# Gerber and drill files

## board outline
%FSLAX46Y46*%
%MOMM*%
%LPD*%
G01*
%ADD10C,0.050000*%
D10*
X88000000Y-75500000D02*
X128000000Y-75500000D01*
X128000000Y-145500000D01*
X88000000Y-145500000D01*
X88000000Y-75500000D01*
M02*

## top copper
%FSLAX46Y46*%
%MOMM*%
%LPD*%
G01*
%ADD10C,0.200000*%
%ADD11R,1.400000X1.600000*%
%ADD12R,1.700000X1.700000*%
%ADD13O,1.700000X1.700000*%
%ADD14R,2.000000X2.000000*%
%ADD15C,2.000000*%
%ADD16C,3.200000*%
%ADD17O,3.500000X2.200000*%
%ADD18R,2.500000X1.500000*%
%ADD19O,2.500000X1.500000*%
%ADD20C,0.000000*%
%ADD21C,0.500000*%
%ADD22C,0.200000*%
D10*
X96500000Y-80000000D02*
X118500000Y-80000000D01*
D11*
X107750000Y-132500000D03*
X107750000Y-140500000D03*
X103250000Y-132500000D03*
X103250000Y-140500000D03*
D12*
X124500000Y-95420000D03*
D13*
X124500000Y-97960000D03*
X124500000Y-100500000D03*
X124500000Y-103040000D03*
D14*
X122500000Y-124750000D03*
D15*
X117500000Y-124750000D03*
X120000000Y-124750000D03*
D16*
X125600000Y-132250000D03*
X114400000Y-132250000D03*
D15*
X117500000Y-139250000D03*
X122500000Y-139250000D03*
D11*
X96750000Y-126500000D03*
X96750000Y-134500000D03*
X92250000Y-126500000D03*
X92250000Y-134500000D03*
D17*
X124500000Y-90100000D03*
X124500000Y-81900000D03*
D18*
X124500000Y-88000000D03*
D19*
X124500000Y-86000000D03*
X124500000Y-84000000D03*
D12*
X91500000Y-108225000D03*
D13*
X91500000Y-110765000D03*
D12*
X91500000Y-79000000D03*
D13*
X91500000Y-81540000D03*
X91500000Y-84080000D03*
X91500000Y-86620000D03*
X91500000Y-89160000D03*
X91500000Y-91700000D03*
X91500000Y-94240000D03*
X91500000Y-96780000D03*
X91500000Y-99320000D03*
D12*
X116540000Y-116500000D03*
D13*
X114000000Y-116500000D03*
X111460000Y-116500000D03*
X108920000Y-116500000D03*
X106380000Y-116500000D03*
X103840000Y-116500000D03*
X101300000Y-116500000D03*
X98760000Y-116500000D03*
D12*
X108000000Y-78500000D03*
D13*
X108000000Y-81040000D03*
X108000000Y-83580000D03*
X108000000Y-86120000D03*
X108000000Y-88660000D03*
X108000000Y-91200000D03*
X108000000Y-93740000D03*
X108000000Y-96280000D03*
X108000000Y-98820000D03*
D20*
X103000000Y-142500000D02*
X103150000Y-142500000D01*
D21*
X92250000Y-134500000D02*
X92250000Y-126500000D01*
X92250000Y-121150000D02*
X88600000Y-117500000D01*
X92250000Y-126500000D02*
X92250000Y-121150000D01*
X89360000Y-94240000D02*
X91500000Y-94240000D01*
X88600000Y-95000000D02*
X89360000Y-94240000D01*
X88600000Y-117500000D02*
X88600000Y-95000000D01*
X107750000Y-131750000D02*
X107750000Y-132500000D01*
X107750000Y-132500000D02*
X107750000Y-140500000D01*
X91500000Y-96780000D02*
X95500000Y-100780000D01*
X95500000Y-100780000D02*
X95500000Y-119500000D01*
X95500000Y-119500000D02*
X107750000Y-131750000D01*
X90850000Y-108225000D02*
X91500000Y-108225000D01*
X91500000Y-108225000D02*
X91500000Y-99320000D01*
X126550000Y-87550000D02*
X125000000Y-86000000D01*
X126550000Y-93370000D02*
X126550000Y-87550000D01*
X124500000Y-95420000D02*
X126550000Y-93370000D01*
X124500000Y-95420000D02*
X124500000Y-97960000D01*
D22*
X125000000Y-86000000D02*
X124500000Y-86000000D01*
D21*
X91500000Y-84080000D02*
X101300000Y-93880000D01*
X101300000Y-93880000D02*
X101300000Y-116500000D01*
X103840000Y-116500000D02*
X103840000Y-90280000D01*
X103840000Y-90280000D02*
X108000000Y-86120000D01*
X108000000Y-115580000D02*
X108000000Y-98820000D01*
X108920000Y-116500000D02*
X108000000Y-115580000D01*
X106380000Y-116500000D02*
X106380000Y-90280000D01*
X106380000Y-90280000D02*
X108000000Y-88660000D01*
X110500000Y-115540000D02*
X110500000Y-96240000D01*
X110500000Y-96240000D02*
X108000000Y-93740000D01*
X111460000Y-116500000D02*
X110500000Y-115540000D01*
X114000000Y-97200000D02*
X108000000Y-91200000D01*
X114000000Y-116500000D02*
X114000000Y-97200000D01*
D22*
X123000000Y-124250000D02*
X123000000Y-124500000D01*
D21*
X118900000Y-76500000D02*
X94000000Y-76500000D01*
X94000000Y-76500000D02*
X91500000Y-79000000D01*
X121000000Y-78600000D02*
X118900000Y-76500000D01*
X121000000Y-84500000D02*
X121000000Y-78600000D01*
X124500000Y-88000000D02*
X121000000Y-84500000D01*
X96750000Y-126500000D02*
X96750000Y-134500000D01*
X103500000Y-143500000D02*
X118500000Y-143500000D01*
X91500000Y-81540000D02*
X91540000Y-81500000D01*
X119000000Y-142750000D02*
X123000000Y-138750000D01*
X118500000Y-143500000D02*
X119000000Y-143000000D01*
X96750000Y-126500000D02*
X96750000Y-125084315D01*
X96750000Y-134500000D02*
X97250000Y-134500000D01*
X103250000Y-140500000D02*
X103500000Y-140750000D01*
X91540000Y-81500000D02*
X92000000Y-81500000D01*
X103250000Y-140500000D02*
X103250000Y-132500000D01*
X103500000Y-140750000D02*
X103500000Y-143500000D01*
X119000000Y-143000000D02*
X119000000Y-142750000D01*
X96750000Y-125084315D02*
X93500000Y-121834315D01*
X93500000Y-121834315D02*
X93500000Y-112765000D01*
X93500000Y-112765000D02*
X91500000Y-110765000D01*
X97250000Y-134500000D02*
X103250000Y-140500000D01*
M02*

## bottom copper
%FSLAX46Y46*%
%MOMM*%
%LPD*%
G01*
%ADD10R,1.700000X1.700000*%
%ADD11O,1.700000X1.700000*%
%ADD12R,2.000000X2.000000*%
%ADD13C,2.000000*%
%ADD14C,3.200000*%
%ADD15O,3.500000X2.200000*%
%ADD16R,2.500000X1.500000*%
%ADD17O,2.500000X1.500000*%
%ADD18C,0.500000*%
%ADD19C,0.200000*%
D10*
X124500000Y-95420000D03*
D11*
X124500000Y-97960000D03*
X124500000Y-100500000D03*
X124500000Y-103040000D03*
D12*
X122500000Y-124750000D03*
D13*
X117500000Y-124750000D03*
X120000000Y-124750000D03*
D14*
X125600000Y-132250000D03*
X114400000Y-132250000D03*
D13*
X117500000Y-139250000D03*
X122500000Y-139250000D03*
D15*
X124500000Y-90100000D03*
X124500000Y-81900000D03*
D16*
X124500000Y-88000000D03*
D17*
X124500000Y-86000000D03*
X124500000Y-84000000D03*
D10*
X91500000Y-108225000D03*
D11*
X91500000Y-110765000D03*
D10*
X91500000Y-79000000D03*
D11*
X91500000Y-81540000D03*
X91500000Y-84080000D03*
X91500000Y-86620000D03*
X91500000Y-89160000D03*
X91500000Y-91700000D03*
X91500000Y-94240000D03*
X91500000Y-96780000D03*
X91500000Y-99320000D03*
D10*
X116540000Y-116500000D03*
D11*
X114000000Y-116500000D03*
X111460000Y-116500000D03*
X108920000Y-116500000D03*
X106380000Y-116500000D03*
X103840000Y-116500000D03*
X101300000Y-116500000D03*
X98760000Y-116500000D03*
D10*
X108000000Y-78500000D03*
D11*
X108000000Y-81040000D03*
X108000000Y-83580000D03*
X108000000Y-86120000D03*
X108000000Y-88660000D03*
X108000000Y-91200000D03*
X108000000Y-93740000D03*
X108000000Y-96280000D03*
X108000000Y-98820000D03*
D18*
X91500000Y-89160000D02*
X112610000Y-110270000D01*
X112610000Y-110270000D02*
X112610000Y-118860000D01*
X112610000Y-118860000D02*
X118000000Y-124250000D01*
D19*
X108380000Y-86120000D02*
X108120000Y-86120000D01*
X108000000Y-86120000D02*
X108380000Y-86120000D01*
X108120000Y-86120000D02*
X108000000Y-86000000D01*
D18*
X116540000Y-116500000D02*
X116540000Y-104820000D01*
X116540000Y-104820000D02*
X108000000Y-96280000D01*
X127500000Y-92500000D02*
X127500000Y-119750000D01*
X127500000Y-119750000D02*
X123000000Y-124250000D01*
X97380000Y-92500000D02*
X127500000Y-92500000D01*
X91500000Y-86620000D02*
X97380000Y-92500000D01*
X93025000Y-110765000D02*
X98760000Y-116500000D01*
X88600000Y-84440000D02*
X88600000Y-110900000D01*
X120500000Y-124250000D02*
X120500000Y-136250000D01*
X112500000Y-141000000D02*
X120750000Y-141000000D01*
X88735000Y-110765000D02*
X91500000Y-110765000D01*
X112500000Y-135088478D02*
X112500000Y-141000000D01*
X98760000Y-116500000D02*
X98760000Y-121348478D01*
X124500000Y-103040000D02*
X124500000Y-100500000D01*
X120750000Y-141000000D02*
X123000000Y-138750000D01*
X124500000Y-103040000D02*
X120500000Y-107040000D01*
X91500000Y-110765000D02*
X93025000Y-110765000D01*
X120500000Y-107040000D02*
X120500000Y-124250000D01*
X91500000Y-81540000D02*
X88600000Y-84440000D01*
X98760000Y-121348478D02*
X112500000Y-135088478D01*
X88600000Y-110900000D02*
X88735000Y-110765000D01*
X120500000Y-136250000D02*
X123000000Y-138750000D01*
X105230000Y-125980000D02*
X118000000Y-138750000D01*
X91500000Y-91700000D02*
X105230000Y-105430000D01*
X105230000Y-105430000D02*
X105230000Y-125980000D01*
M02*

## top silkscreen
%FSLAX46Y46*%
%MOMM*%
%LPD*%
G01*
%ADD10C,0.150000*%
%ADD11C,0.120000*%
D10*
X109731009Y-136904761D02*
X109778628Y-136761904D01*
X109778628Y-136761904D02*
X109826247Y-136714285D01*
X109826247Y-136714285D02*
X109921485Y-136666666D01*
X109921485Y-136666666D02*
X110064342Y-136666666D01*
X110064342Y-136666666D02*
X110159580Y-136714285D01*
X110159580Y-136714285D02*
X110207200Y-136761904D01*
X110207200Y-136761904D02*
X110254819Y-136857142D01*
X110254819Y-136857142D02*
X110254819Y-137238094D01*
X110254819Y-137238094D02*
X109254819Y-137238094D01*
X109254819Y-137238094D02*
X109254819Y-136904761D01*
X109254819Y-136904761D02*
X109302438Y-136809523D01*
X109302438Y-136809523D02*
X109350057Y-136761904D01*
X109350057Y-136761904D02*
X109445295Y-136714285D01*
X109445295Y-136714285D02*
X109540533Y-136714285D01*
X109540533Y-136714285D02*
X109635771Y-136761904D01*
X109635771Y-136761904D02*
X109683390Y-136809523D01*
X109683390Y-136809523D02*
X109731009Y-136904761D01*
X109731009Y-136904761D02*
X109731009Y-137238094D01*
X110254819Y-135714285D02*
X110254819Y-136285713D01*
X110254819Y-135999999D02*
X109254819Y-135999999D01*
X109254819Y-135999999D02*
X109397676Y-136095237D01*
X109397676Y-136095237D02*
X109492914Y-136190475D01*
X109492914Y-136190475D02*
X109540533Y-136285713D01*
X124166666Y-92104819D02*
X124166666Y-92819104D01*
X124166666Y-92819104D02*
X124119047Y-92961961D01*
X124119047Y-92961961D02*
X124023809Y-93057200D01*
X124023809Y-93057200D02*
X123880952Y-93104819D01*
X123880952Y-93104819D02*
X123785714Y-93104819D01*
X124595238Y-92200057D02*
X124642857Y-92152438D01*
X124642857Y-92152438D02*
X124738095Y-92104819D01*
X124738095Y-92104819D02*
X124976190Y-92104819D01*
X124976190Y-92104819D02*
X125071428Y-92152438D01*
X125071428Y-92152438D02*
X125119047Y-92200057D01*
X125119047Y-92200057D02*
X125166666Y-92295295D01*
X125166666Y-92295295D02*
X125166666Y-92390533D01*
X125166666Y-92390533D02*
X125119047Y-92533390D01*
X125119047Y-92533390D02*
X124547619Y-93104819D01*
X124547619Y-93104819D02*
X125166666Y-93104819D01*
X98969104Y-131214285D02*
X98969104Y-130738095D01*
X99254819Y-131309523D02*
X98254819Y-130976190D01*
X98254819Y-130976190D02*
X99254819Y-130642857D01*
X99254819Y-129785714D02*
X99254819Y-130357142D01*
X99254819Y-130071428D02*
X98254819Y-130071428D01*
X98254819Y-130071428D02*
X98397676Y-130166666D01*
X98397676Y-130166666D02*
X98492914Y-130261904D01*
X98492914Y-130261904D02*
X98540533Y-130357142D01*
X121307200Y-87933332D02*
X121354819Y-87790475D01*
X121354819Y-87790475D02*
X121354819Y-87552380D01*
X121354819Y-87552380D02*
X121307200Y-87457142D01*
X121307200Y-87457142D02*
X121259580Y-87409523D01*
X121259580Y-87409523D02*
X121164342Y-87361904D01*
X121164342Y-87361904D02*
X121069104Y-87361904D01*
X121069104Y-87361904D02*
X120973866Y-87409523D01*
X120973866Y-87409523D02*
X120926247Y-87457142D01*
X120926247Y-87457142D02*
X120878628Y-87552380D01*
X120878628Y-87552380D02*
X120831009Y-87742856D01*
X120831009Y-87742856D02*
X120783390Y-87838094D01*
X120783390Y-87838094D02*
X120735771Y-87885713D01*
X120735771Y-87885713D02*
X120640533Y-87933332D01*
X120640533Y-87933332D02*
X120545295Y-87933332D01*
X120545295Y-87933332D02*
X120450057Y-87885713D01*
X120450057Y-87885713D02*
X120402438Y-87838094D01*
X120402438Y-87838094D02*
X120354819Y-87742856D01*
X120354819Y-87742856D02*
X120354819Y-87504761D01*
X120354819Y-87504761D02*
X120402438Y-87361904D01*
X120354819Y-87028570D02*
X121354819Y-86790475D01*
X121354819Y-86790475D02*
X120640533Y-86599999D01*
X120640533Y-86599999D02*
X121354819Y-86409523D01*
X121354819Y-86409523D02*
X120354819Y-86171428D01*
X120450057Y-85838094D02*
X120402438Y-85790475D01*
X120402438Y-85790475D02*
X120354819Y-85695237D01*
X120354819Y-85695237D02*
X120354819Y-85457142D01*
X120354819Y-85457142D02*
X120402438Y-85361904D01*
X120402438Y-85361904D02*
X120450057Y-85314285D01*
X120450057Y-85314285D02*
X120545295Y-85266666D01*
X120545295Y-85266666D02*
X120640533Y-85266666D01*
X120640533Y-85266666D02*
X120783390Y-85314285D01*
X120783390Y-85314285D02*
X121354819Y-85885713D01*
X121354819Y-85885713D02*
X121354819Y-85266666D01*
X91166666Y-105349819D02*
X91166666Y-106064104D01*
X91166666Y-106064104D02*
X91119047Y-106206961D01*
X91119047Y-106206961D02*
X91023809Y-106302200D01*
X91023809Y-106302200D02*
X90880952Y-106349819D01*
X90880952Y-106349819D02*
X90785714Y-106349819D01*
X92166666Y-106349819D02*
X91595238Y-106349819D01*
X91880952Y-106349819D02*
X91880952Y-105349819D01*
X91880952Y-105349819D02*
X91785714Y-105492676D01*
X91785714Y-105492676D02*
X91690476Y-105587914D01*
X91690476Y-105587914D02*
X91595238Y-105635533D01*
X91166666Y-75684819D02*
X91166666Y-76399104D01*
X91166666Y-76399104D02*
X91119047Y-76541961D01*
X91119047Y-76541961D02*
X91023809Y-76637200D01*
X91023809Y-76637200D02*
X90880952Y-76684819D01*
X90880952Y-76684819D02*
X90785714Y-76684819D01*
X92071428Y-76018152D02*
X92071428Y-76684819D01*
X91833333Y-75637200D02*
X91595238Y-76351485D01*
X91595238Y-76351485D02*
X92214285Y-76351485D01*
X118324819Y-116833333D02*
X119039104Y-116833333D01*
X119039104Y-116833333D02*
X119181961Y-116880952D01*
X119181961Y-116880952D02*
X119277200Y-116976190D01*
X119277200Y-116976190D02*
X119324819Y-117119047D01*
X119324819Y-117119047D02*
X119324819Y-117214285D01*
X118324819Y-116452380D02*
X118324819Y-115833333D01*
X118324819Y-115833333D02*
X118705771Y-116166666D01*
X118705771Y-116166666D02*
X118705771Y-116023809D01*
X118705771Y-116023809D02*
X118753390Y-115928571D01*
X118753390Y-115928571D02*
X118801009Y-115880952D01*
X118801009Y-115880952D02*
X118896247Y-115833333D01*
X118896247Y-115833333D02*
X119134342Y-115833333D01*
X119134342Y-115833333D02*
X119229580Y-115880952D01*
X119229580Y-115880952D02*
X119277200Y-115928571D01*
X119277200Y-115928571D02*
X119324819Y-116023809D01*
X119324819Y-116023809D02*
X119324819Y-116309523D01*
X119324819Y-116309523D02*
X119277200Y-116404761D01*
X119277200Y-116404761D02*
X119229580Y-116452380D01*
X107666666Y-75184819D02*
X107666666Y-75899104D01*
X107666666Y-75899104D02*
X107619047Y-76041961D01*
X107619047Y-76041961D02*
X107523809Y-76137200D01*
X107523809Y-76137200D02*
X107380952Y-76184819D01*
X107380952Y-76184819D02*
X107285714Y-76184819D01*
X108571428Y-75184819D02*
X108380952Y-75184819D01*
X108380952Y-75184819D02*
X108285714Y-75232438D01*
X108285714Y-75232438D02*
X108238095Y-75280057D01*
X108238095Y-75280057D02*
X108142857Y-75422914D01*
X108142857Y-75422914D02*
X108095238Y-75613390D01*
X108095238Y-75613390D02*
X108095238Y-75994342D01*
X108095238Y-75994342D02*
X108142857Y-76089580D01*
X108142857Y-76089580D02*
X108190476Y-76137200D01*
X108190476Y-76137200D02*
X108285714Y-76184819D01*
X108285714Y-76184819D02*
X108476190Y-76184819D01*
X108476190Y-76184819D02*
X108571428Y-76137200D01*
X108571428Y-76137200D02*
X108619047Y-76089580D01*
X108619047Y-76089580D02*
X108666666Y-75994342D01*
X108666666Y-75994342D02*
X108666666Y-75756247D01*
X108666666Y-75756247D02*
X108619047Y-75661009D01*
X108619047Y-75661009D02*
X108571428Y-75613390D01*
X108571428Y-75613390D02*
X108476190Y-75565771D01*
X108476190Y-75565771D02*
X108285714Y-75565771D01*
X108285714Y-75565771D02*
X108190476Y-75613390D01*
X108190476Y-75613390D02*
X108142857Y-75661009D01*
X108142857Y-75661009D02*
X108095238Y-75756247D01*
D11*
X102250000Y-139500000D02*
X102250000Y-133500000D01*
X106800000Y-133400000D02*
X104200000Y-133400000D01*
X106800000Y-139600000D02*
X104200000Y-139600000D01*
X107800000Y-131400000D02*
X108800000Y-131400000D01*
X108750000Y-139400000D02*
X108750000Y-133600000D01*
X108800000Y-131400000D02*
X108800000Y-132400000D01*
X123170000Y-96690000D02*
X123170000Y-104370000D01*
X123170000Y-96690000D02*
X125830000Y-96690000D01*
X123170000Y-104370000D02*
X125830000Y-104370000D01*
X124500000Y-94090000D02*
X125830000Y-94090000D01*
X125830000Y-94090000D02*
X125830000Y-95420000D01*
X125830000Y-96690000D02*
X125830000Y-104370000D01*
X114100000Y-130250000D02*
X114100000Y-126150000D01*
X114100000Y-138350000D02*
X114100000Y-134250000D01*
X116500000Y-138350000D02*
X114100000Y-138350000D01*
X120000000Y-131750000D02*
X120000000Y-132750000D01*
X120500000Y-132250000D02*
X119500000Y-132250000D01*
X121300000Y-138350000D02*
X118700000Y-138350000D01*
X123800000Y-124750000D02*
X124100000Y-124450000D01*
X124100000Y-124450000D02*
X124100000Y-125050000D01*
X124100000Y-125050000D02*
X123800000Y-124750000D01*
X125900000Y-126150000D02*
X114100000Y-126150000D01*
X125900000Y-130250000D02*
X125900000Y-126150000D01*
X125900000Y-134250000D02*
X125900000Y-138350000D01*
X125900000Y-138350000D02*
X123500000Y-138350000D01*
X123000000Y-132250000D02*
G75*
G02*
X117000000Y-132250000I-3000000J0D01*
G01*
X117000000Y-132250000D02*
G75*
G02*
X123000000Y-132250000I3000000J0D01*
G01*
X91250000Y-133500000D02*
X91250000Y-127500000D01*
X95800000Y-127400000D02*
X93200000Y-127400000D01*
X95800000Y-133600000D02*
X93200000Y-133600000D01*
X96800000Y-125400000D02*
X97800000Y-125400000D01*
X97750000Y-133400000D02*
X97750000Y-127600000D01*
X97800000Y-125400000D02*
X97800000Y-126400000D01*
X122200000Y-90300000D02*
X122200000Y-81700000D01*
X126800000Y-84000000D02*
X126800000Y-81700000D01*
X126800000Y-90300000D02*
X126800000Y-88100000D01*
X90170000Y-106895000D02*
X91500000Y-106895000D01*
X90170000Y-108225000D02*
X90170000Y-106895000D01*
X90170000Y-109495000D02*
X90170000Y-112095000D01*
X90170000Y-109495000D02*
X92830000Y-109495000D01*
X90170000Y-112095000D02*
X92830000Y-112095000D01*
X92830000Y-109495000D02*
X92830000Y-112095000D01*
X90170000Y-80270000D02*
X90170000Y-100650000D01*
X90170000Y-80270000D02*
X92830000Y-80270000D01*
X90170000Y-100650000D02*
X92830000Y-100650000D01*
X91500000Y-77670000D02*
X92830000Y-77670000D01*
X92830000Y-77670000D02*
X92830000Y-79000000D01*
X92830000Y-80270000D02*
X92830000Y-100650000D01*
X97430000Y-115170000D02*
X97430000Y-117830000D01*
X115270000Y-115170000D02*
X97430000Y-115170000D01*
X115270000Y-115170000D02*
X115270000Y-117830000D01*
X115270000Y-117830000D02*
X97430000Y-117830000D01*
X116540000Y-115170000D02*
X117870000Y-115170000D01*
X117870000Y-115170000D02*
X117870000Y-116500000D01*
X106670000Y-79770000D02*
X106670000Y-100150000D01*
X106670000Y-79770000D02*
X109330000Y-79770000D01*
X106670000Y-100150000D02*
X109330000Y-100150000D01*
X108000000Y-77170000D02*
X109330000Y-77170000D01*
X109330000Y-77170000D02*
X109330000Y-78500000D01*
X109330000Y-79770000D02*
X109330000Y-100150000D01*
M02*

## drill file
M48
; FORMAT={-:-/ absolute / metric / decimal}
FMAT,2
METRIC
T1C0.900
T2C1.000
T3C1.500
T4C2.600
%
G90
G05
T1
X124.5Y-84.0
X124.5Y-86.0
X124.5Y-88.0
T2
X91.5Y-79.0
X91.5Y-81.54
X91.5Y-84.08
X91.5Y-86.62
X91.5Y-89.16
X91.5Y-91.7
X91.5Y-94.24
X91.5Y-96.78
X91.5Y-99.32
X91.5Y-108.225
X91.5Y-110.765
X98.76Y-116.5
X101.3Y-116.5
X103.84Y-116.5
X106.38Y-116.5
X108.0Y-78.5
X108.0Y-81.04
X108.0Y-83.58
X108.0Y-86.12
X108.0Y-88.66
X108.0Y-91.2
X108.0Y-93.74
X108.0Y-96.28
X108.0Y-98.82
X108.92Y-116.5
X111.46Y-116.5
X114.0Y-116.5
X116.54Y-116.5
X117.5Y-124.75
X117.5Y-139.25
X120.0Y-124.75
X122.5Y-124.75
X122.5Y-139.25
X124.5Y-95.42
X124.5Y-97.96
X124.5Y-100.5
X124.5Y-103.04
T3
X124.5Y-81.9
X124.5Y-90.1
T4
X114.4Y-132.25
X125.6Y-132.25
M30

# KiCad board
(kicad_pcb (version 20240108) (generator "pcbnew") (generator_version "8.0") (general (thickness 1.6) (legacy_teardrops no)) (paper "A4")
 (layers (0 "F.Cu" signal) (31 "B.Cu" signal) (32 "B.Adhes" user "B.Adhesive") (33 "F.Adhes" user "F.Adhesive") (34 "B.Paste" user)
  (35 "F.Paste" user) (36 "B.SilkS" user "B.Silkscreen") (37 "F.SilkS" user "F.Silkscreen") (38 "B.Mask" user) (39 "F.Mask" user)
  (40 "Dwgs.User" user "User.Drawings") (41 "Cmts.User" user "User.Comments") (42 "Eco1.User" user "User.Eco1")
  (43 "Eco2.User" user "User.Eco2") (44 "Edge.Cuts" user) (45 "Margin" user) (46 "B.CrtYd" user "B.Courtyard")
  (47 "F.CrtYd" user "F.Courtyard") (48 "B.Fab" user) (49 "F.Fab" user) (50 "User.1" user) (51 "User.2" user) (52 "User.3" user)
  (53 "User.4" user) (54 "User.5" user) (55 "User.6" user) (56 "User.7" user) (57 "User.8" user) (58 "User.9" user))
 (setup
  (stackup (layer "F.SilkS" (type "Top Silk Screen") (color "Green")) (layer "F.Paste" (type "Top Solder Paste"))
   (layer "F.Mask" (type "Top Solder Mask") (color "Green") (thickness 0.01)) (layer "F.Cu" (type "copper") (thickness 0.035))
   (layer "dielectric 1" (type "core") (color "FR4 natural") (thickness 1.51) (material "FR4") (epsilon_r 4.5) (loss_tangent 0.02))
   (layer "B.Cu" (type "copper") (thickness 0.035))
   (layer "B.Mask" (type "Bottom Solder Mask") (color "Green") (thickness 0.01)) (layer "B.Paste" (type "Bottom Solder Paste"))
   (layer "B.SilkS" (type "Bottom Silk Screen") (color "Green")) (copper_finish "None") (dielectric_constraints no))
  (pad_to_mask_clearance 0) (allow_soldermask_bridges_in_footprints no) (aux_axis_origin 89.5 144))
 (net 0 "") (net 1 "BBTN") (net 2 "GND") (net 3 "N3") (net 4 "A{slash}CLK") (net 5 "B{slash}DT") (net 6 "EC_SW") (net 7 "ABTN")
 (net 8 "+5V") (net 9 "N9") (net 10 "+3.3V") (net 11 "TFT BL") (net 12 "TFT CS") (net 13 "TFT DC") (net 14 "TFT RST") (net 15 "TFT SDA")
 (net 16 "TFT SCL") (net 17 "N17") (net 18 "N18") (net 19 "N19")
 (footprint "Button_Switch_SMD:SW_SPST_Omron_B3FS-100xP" (layer "F.Cu") (at 105.5 136.5 -90)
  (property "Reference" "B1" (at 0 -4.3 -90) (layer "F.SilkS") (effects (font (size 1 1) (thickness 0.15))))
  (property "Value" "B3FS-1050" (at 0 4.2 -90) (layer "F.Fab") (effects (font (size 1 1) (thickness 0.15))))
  (fp_line (start 3 3.25) (end -3 3.25) (stroke (width 0.12) (type solid)) (layer "F.SilkS"))
  (fp_line (start -3.1 -1.3) (end -3.1 1.3) (stroke (width 0.12) (type solid)) (layer "F.SilkS"))
  (fp_line (start 3.1 -1.3) (end 3.1 1.3) (stroke (width 0.12) (type solid)) (layer "F.SilkS"))
  (fp_line (start -5.1 -2.3) (end -5.1 -3.3) (stroke (width 0.12) (type solid)) (layer "F.SilkS"))
  (fp_line (start 2.9 -3.25) (end -2.9 -3.25) (stroke (width 0.12) (type solid)) (layer "F.SilkS"))
  (fp_line (start -5.1 -3.3) (end -4.1 -3.3) (stroke (width 0.12) (type solid)) (layer "F.SilkS"))
  (pad "1" smd rect (at -4 -2.25 90) (size 1.6 1.4) (layers "F.Cu" "F.Paste" "F.Mask") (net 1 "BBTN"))
  (pad "1" smd rect (at 4 -2.25 90) (size 1.6 1.4) (layers "F.Cu" "F.Paste" "F.Mask") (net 1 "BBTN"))
  (pad "2" smd rect (at -4 2.25 90) (size 1.6 1.4) (layers "F.Cu" "F.Paste" "F.Mask") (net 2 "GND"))
  (pad "2" smd rect (at 4 2.25 90) (size 1.6 1.4) (layers "F.Cu" "F.Paste" "F.Mask") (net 2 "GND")))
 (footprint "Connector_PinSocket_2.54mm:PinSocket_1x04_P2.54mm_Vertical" (layer "F.Cu") (at 124.5 95.42)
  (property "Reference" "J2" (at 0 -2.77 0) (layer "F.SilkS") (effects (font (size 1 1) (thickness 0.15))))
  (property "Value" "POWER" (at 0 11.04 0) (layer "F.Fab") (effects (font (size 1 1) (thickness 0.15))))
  (fp_line (start -1.33 1.27) (end -1.33 8.95) (stroke (width 0.12) (type solid)) (layer "F.SilkS"))
  (fp_line (start -1.33 1.27) (end 1.33 1.27) (stroke (width 0.12) (type solid)) (layer "F.SilkS"))
  (fp_line (start -1.33 8.95) (end 1.33 8.95) (stroke (width 0.12) (type solid)) (layer "F.SilkS"))
  (fp_line (start 0 -1.33) (end 1.33 -1.33) (stroke (width 0.12) (type solid)) (layer "F.SilkS"))
  (fp_line (start 1.33 -1.33) (end 1.33 0) (stroke (width 0.12) (type solid)) (layer "F.SilkS"))
  (fp_line (start 1.33 1.27) (end 1.33 8.95) (stroke (width 0.12) (type solid)) (layer "F.SilkS"))
  (pad "1" thru_hole rect (at 0 0) (size 1.7 1.7) (drill 1) (layers "*.Cu" "*.Mask") (remove_unused_layers no) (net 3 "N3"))
  (pad "2" thru_hole oval (at 0 2.54) (size 1.7 1.7) (drill 1) (layers "*.Cu" "*.Mask") (remove_unused_layers no) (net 3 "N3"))
  (pad "3" thru_hole oval (at 0 5.08) (size 1.7 1.7) (drill 1) (layers "*.Cu" "*.Mask") (remove_unused_layers no) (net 2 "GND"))
  (pad "4" thru_hole oval (at 0 7.62) (size 1.7 1.7) (drill 1) (layers "*.Cu" "*.Mask") (remove_unused_layers no) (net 2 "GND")))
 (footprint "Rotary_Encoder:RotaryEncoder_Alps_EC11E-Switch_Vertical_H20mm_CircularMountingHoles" (layer "F.Cu") (at 122.5 124.75 -90)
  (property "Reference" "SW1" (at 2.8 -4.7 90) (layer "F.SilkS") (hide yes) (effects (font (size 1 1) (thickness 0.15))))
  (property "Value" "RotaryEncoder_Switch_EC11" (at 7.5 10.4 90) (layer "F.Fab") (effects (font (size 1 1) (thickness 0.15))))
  (fp_line (start 5.5 8.4) (end 1.4 8.4) (stroke (width 0.12) (type solid)) (layer "F.SilkS"))
  (fp_line (start 13.6 8.4) (end 9.5 8.4) (stroke (width 0.12) (type solid)) (layer "F.SilkS"))
  (fp_line (start 13.6 6) (end 13.6 8.4) (stroke (width 0.12) (type solid)) (layer "F.SilkS"))
  (fp_line (start 7 2.5) (end 8 2.5) (stroke (width 0.12) (type solid)) (layer "F.SilkS"))
  (fp_line (start 7.5 2) (end 7.5 3) (stroke (width 0.12) (type solid)) (layer "F.SilkS"))
  (fp_line (start 13.6 1.2) (end 13.6 3.8) (stroke (width 0.12) (type solid)) (layer "F.SilkS"))
  (fp_line (start 0 -1.3) (end -0.3 -1.6) (stroke (width 0.12) (type solid)) (layer "F.SilkS"))
  (fp_line (start -0.3 -1.6) (end 0.3 -1.6) (stroke (width 0.12) (type solid)) (layer "F.SilkS"))
  (fp_line (start 0.3 -1.6) (end 0 -1.3) (stroke (width 0.12) (type solid)) (layer "F.SilkS"))
  (fp_line (start 1.4 -3.4) (end 1.4 8.4) (stroke (width 0.12) (type solid)) (layer "F.SilkS"))
  (fp_line (start 5.5 -3.4) (end 1.4 -3.4) (stroke (width 0.12) (type solid)) (layer "F.SilkS"))
  (fp_line (start 9.5 -3.4) (end 13.6 -3.4) (stroke (width 0.12) (type solid)) (layer "F.SilkS"))
  (fp_line (start 13.6 -3.4) (end 13.6 -1) (stroke (width 0.12) (type solid)) (layer "F.SilkS"))
  (fp_circle (center 7.5 2.5) (end 10.5 2.5) (stroke (width 0.12) (type solid)) (fill none) (layer "F.SilkS"))
  (pad "A" thru_hole rect (at 0 0 270) (size 2 2) (drill 1) (layers "*.Cu" "*.Mask") (remove_unused_layers no) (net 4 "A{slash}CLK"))
  (pad "B" thru_hole circle (at 0 5 270) (size 2 2) (drill 1) (layers "*.Cu" "*.Mask") (remove_unused_layers no) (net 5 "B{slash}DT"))
  (pad "C" thru_hole circle (at 0 2.5 270) (size 2 2) (drill 1) (layers "*.Cu" "*.Mask") (remove_unused_layers no) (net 2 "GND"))
  (pad "MP" thru_hole circle (at 7.5 -3.1 270) (size 3.2 3.2) (drill 2.6) (layers "*.Cu" "*.Mask") (remove_unused_layers no))
  (pad "MP" thru_hole circle (at 7.5 8.1 270) (size 3.2 3.2) (drill 2.6) (layers "*.Cu" "*.Mask") (remove_unused_layers no))
  (pad "S1" thru_hole circle (at 14.5 5 270) (size 2 2) (drill 1) (layers "*.Cu" "*.Mask") (remove_unused_layers no) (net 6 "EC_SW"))
  (pad "S2" thru_hole circle (at 14.5 0 270) (size 2 2) (drill 1) (layers "*.Cu" "*.Mask") (remove_unused_layers no) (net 2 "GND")))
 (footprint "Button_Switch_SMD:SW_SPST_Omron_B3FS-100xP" (layer "F.Cu") (at 94.5 130.5 -90)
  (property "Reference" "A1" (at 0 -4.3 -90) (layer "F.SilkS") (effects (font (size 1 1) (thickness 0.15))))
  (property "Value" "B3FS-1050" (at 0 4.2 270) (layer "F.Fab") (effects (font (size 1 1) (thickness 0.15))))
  (fp_line (start 3 3.25) (end -3 3.25) (stroke (width 0.12) (type solid)) (layer "F.SilkS"))
  (fp_line (start -3.1 -1.3) (end -3.1 1.3) (stroke (width 0.12) (type solid)) (layer "F.SilkS"))
  (fp_line (start 3.1 -1.3) (end 3.1 1.3) (stroke (width 0.12) (type solid)) (layer "F.SilkS"))
  (fp_line (start -5.1 -2.3) (end -5.1 -3.3) (stroke (width 0.12) (type solid)) (layer "F.SilkS"))
  (fp_line (start 2.9 -3.25) (end -2.9 -3.25) (stroke (width 0.12) (type solid)) (layer "F.SilkS"))
  (fp_line (start -5.1 -3.3) (end -4.1 -3.3) (stroke (width 0.12) (type solid)) (layer "F.SilkS"))
  (pad "1" smd rect (at -4 -2.25 90) (size 1.6 1.4) (layers "F.Cu" "F.Paste" "F.Mask") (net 2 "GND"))
  (pad "1" smd rect (at 4 -2.25 90) (size 1.6 1.4) (layers "F.Cu" "F.Paste" "F.Mask") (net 2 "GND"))
  (pad "2" smd rect (at -4 2.25 90) (size 1.6 1.4) (layers "F.Cu" "F.Paste" "F.Mask") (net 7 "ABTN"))
  (pad "2" smd rect (at 4 2.25 90) (size 1.6 1.4) (layers "F.Cu" "F.Paste" "F.Mask") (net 7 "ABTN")))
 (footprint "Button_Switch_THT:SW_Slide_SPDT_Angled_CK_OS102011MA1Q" (layer "F.Cu") (at 124.5 88 90)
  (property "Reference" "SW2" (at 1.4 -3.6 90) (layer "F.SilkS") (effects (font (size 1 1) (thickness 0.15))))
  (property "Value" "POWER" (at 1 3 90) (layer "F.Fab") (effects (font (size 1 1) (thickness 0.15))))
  (fp_line (start -2.3 -2.3) (end 6.3 -2.3) (stroke (width 0.12) (type solid)) (layer "F.SilkS"))
  (fp_line (start 4 2.3) (end 6.3 2.3) (stroke (width 0.12) (type solid)) (layer "F.SilkS"))
  (fp_line (start -2.3 2.3) (end -0.1 2.3) (stroke (width 0.12) (type solid)) (layer "F.SilkS"))
  (pad "" thru_hole oval (at -2.1 0 90) (size 2.2 3.5) (drill 1.5) (layers "*.Cu" "*.Mask") (remove_unused_layers no))
  (pad "" thru_hole oval (at 6.1 0 90) (size 2.2 3.5) (drill 1.5) (layers "*.Cu" "*.Mask") (remove_unused_layers no))
  (pad "1" thru_hole rect (at 0 0 90) (size 1.5 2.5) (drill 0.9) (layers "*.Cu" "*.Mask") (remove_unused_layers no) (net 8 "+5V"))
  (pad "2" thru_hole oval (at 2 0 90) (size 1.5 2.5) (drill 0.9) (layers "*.Cu" "*.Mask") (remove_unused_layers no) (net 3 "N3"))
  (pad "3" thru_hole oval (at 4 0 90) (size 1.5 2.5) (drill 0.9) (layers "*.Cu" "*.Mask") (remove_unused_layers no)))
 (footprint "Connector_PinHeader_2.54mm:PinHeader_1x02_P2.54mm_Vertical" (layer "F.Cu") (at 91.5 108.225)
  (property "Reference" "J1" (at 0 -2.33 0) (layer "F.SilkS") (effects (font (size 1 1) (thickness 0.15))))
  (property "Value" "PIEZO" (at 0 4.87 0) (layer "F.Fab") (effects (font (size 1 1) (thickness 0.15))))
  (fp_line (start -1.33 -1.33) (end 0 -1.33) (stroke (width 0.12) (type solid)) (layer "F.SilkS"))
  (fp_line (start -1.33 0) (end -1.33 -1.33) (stroke (width 0.12) (type solid)) (layer "F.SilkS"))
  (fp_line (start -1.33 1.27) (end -1.33 3.87) (stroke (width 0.12) (type solid)) (layer "F.SilkS"))
  (fp_line (start -1.33 1.27) (end 1.33 1.27) (stroke (width 0.12) (type solid)) (layer "F.SilkS"))
  (fp_line (start -1.33 3.87) (end 1.33 3.87) (stroke (width 0.12) (type solid)) (layer "F.SilkS"))
  (fp_line (start 1.33 1.27) (end 1.33 3.87) (stroke (width 0.12) (type solid)) (layer "F.SilkS"))
  (pad "1" thru_hole rect (at 0 0) (size 1.7 1.7) (drill 1) (layers "*.Cu" "*.Mask") (remove_unused_layers no) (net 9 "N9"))
  (pad "2" thru_hole oval (at 0 2.54) (size 1.7 1.7) (drill 1) (layers "*.Cu" "*.Mask") (remove_unused_layers no) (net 2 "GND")))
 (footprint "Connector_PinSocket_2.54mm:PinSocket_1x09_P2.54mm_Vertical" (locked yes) (layer "F.Cu") (at 91.5 79)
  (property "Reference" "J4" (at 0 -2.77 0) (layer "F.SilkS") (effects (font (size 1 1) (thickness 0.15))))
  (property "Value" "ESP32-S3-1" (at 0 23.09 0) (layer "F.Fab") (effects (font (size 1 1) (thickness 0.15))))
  (fp_line (start -1.33 1.27) (end -1.33 21.65) (stroke (width 0.12) (type solid)) (layer "F.SilkS"))
  (fp_line (start -1.33 1.27) (end 1.33 1.27) (stroke (width 0.12) (type solid)) (layer "F.SilkS"))
  (fp_line (start -1.33 21.65) (end 1.33 21.65) (stroke (width 0.12) (type solid)) (layer "F.SilkS"))
  (fp_line (start 0 -1.33) (end 1.33 -1.33) (stroke (width 0.12) (type solid)) (layer "F.SilkS"))
  (fp_line (start 1.33 -1.33) (end 1.33 0) (stroke (width 0.12) (type solid)) (layer "F.SilkS"))
  (fp_line (start 1.33 1.27) (end 1.33 21.65) (stroke (width 0.12) (type solid)) (layer "F.SilkS"))
  (pad "1" thru_hole rect (at 0 0) (size 1.7 1.7) (drill 1) (layers "*.Cu" "*.Mask") (remove_unused_layers no) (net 8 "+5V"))
  (pad "2" thru_hole oval (at 0 2.54) (size 1.7 1.7) (drill 1) (layers "*.Cu" "*.Mask") (remove_unused_layers no) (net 2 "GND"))
  (pad "3" thru_hole oval (at 0 5.08) (size 1.7 1.7) (drill 1) (layers "*.Cu" "*.Mask") (remove_unused_layers no) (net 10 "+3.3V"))
  (pad "4" thru_hole oval (at 0 7.62) (size 1.7 1.7) (drill 1) (layers "*.Cu" "*.Mask") (remove_unused_layers no) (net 4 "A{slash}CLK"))
  (pad "5" thru_hole oval (at 0 10.16) (size 1.7 1.7) (drill 1) (layers "*.Cu" "*.Mask") (remove_unused_layers no) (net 5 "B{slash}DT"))
  (pad "6" thru_hole oval (at 0 12.7) (size 1.7 1.7) (drill 1) (layers "*.Cu" "*.Mask") (remove_unused_layers no) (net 6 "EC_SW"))
  (pad "7" thru_hole oval (at 0 15.24) (size 1.7 1.7) (drill 1) (layers "*.Cu" "*.Mask") (remove_unused_layers no) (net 7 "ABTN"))
  (pad "8" thru_hole oval (at 0 17.78) (size 1.7 1.7) (drill 1) (layers "*.Cu" "*.Mask") (remove_unused_layers no) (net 1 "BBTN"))
  (pad "9" thru_hole oval (at 0 20.32) (size 1.7 1.7) (drill 1) (layers "*.Cu" "*.Mask") (remove_unused_layers no) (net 9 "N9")))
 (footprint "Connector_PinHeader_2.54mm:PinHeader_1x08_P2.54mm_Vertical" (layer "F.Cu") (at 116.54 116.5 -90)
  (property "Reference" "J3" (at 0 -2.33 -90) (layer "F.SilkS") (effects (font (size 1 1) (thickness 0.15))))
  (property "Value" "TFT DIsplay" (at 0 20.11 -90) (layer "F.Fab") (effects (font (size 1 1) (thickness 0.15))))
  (fp_line (start -1.33 19.11) (end 1.33 19.11) (stroke (width 0.12) (type solid)) (layer "F.SilkS"))
  (fp_line (start -1.33 1.27) (end -1.33 19.11) (stroke (width 0.12) (type solid)) (layer "F.SilkS"))
  (fp_line (start -1.33 1.27) (end 1.33 1.27) (stroke (width 0.12) (type solid)) (layer "F.SilkS"))
  (fp_line (start 1.33 1.27) (end 1.33 19.11) (stroke (width 0.12) (type solid)) (layer "F.SilkS"))
  (fp_line (start -1.33 0) (end -1.33 -1.33) (stroke (width 0.12) (type solid)) (layer "F.SilkS"))
  (fp_line (start -1.33 -1.33) (end 0 -1.33) (stroke (width 0.12) (type solid)) (layer "F.SilkS"))
  (pad "1" thru_hole rect (at 0 0 270) (size 1.7 1.7) (drill 1) (layers "*.Cu" "*.Mask") (remove_unused_layers no) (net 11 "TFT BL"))
  (pad "2" thru_hole oval (at 0 2.54 270) (size 1.7 1.7) (drill 1) (layers "*.Cu" "*.Mask") (remove_unused_layers no) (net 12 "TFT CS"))
  (pad "3" thru_hole oval (at 0 5.08 270) (size 1.7 1.7) (drill 1) (layers "*.Cu" "*.Mask") (remove_unused_layers no) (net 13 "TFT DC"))
  (pad "4" thru_hole oval (at 0 7.62 270) (size 1.7 1.7) (drill 1) (layers "*.Cu" "*.Mask") (remove_unused_layers no) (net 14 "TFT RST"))
  (pad "5" thru_hole oval (at 0 10.16 270) (size 1.7 1.7) (drill 1) (layers "*.Cu" "*.Mask") (remove_unused_layers no) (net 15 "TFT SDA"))
  (pad "6" thru_hole oval (at 0 12.7 270) (size 1.7 1.7) (drill 1) (layers "*.Cu" "*.Mask") (remove_unused_layers no) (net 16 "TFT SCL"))
  (pad "7" thru_hole oval (at 0 15.24 270) (size 1.7 1.7) (drill 1) (layers "*.Cu" "*.Mask") (remove_unused_layers no) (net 10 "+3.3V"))
  (pad "8" thru_hole oval (at 0 17.78 270) (size 1.7 1.7) (drill 1) (layers "*.Cu" "*.Mask") (remove_unused_layers no) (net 2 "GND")))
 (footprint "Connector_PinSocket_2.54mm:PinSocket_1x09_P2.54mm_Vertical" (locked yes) (layer "F.Cu") (at 108 78.5)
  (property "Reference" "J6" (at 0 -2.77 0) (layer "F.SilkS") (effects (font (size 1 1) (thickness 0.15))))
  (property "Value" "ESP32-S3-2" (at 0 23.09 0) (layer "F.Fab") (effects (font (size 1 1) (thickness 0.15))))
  (fp_line (start -1.33 1.27) (end -1.33 21.65) (stroke (width 0.12) (type solid)) (layer "F.SilkS"))
  (fp_line (start -1.33 1.27) (end 1.33 1.27) (stroke (width 0.12) (type solid)) (layer "F.SilkS"))
  (fp_line (start -1.33 21.65) (end 1.33 21.65) (stroke (width 0.12) (type solid)) (layer "F.SilkS"))
  (fp_line (start 0 -1.33) (end 1.33 -1.33) (stroke (width 0.12) (type solid)) (layer "F.SilkS"))
  (fp_line (start 1.33 -1.33) (end 1.33 0) (stroke (width 0.12) (type solid)) (layer "F.SilkS"))
  (fp_line (start 1.33 1.27) (end 1.33 21.65) (stroke (width 0.12) (type solid)) (layer "F.SilkS"))
  (pad "1" thru_hole rect (at 0 0) (size 1.7 1.7) (drill 1) (layers "*.Cu" "*.Mask") (remove_unused_layers no) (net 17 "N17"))
  (pad "2" thru_hole oval (at 0 2.54) (size 1.7 1.7) (drill 1) (layers "*.Cu" "*.Mask") (remove_unused_layers no) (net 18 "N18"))
  (pad "3" thru_hole oval (at 0 5.08) (size 1.7 1.7) (drill 1) (layers "*.Cu" "*.Mask") (remove_unused_layers no) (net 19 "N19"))
  (pad "4" thru_hole oval (at 0 7.62) (size 1.7 1.7) (drill 1) (layers "*.Cu" "*.Mask") (remove_unused_layers no) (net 16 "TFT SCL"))
  (pad "5" thru_hole oval (at 0 10.16) (size 1.7 1.7) (drill 1) (layers "*.Cu" "*.Mask") (remove_unused_layers no) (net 15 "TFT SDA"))
  (pad "6" thru_hole oval (at 0 12.7) (size 1.7 1.7) (drill 1) (layers "*.Cu" "*.Mask") (remove_unused_layers no) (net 12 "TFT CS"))
  (pad "7" thru_hole oval (at 0 15.24) (size 1.7 1.7) (drill 1) (layers "*.Cu" "*.Mask") (remove_unused_layers no) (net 13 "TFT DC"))
  (pad "8" thru_hole oval (at 0 17.78) (size 1.7 1.7) (drill 1) (layers "*.Cu" "*.Mask") (remove_unused_layers no) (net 11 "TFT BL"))
  (pad "9" thru_hole oval (at 0 20.32) (size 1.7 1.7) (drill 1) (layers "*.Cu" "*.Mask") (remove_unused_layers no) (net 14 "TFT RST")))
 (gr_line (start 96.5 80) (end 118.5 80) (locked yes) (stroke (width 0.2) (type default)) (layer "F.Cu"))
 (gr_rect (start 88 75.5) (end 128 145.5) (stroke (width 0.05) (type default)) (fill none) (layer "Edge.Cuts"))
 (segment (start 103 142.5) (end 103.15 142.5) (width 0) (layer "F.Cu") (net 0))
 (segment (start 92.25 134.5) (end 92.25 126.5) (width 0.5) (layer "F.Cu") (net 7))
 (segment (start 92.25 121.15) (end 88.6 117.5) (width 0.5) (layer "F.Cu") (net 7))
 (segment (start 92.25 126.5) (end 92.25 121.15) (width 0.5) (layer "F.Cu") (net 7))
 (segment (start 89.36 94.24) (end 91.5 94.24) (width 0.5) (layer "F.Cu") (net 7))
 (segment (start 88.6 95) (end 89.36 94.24) (width 0.5) (layer "F.Cu") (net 7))
 (segment (start 88.6 117.5) (end 88.6 95) (width 0.5) (layer "F.Cu") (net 7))
 (segment (start 91.5 89.16) (end 112.61 110.27) (width 0.5) (layer "B.Cu") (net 5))
 (segment (start 112.61 110.27) (end 112.61 118.86) (width 0.5) (layer "B.Cu") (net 5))
 (segment (start 112.61 118.86) (end 118 124.25) (width 0.5) (layer "B.Cu") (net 5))
 (segment (start 107.75 131.75) (end 107.75 132.5) (width 0.5) (layer "F.Cu") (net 1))
 (segment (start 107.75 132.5) (end 107.75 140.5) (width 0.5) (layer "F.Cu") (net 1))
 (segment (start 91.5 96.78) (end 95.5 100.78) (width 0.5) (layer "F.Cu") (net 1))
 (segment (start 95.5 100.78) (end 95.5 119.5) (width 0.5) (layer "F.Cu") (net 1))
 (segment (start 95.5 119.5) (end 107.75 131.75) (width 0.5) (layer "F.Cu") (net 1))
 (segment (start 90.85 108.225) (end 91.5 108.225) (width 0.5) (layer "F.Cu") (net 9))
 (segment (start 91.5 108.225) (end 91.5 99.32) (width 0.5) (layer "F.Cu") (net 9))
 (segment (start 126.55 87.55) (end 125 86) (width 0.5) (layer "F.Cu") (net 3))
 (segment (start 126.55 93.37) (end 126.55 87.55) (width 0.5) (layer "F.Cu") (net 3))
 (segment (start 124.5 95.42) (end 126.55 93.37) (width 0.5) (layer "F.Cu") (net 3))
 (segment (start 124.5 95.42) (end 124.5 97.96) (width 0.5) (layer "F.Cu") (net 3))
 (segment (start 125 86) (end 124.5 86) (width 0.2) (layer "F.Cu") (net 3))
 (segment (start 91.5 84.08) (end 101.3 93.88) (width 0.5) (layer "F.Cu") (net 10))
 (segment (start 101.3 93.88) (end 101.3 116.5) (width 0.5) (layer "F.Cu") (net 10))
 (segment (start 103.84 116.5) (end 103.84 90.28) (width 0.5) (layer "F.Cu") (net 16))
 (segment (start 103.84 90.28) (end 108 86.12) (width 0.5) (layer "F.Cu") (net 16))
 (segment (start 108.38 86.12) (end 108.12 86.12) (width 0.2) (layer "B.Cu") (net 16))
 (segment (start 108 86.12) (end 108.38 86.12) (width 0.2) (layer "B.Cu") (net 16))
 (segment (start 108.12 86.12) (end 108 86) (width 0.2) (layer "B.Cu") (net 16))
 (segment (start 108 115.58) (end 108 98.82) (width 0.5) (layer "F.Cu") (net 14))
 (segment (start 108.92 116.5) (end 108 115.58) (width 0.5) (layer "F.Cu") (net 14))
 (segment (start 106.38 116.5) (end 106.38 90.28) (width 0.5) (layer "F.Cu") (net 15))
 (segment (start 106.38 90.28) (end 108 88.66) (width 0.5) (layer "F.Cu") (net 15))
 (segment (start 110.5 115.54) (end 110.5 96.24) (width 0.5) (layer "F.Cu") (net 13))
 (segment (start 110.5 96.24) (end 108 93.74) (width 0.5) (layer "F.Cu") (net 13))
 (segment (start 111.46 116.5) (end 110.5 115.54) (width 0.5) (layer "F.Cu") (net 13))
 (segment (start 116.54 116.5) (end 116.54 104.82) (width 0.5) (layer "B.Cu") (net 11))
 (segment (start 116.54 104.82) (end 108 96.28) (width 0.5) (layer "B.Cu") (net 11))
 (segment (start 114 97.2) (end 108 91.2) (width 0.5) (layer "F.Cu") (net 12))
 (segment (start 114 116.5) (end 114 97.2) (width 0.5) (layer "F.Cu") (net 12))
 (segment (start 123 124.25) (end 123 124.5) (width 0.2) (layer "F.Cu") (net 4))
 (segment (start 127.5 92.5) (end 127.5 119.75) (width 0.5) (layer "B.Cu") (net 4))
 (segment (start 127.5 119.75) (end 123 124.25) (width 0.5) (layer "B.Cu") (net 4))
 (segment (start 97.38 92.5) (end 127.5 92.5) (width 0.5) (layer "B.Cu") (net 4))
 (segment (start 91.5 86.62) (end 97.38 92.5) (width 0.5) (layer "B.Cu") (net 4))
 (segment (start 118.9 76.5) (end 94 76.5) (width 0.5) (layer "F.Cu") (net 8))
 (segment (start 94 76.5) (end 91.5 79) (width 0.5) (layer "F.Cu") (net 8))
 (segment (start 121 78.6) (end 118.9 76.5) (width 0.5) (layer "F.Cu") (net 8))
 (segment (start 121 84.5) (end 121 78.6) (width 0.5) (layer "F.Cu") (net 8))
 (segment (start 124.5 88) (end 121 84.5) (width 0.5) (layer "F.Cu") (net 8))
 (segment (start 96.75 126.5) (end 96.75 134.5) (width 0.5) (layer "F.Cu") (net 2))
 (segment (start 103.5 143.5) (end 118.5 143.5) (width 0.5) (layer "F.Cu") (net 2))
 (segment (start 91.5 81.54) (end 91.54 81.5) (width 0.5) (layer "F.Cu") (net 2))
 (segment (start 119 142.75) (end 123 138.75) (width 0.5) (layer "F.Cu") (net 2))
 (segment (start 118.5 143.5) (end 119 143) (width 0.5) (layer "F.Cu") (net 2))
 (segment (start 96.75 126.5) (end 96.75 125.084315) (width 0.5) (layer "F.Cu") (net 2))
 (segment (start 96.75 134.5) (end 97.25 134.5) (width 0.5) (layer "F.Cu") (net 2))
 (segment (start 103.25 140.5) (end 103.5 140.75) (width 0.5) (layer "F.Cu") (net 2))
 (segment (start 91.54 81.5) (end 92 81.5) (width 0.5) (layer "F.Cu") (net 2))
 (segment (start 103.25 140.5) (end 103.25 132.5) (width 0.5) (layer "F.Cu") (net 2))
 (segment (start 103.5 140.75) (end 103.5 143.5) (width 0.5) (layer "F.Cu") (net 2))
 (segment (start 119 143) (end 119 142.75) (width 0.5) (layer "F.Cu") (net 2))
 (segment (start 96.75 125.084315) (end 93.5 121.834315) (width 0.5) (layer "F.Cu") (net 2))
 (segment (start 93.5 121.834315) (end 93.5 112.765) (width 0.5) (layer "F.Cu") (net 2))
 (segment (start 93.5 112.765) (end 91.5 110.765) (width 0.5) (layer "F.Cu") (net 2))
 (segment (start 97.25 134.5) (end 103.25 140.5) (width 0.5) (layer "F.Cu") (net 2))
 (segment (start 93.025 110.765) (end 98.76 116.5) (width 0.5) (layer "B.Cu") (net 2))
 (segment (start 88.6 84.44) (end 88.6 110.9) (width 0.5) (layer "B.Cu") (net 2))
 (segment (start 120.5 124.25) (end 120.5 136.25) (width 0.5) (layer "B.Cu") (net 2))
 (segment (start 112.5 141) (end 120.75 141) (width 0.5) (layer "B.Cu") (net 2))
 (segment (start 88.735 110.765) (end 91.5 110.765) (width 0.5) (layer "B.Cu") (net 2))
 (segment (start 112.5 135.088478) (end 112.5 141) (width 0.5) (layer "B.Cu") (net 2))
 (segment (start 98.76 116.5) (end 98.76 121.348478) (width 0.5) (layer "B.Cu") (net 2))
 (segment (start 124.5 103.04) (end 124.5 100.5) (width 0.5) (layer "B.Cu") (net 2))
 (segment (start 120.75 141) (end 123 138.75) (width 0.5) (layer "B.Cu") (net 2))
 (segment (start 124.5 103.04) (end 120.5 107.04) (width 0.5) (layer "B.Cu") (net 2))
 (segment (start 91.5 110.765) (end 93.025 110.765) (width 0.5) (layer "B.Cu") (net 2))
 (segment (start 120.5 107.04) (end 120.5 124.25) (width 0.5) (layer "B.Cu") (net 2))
 (segment (start 91.5 81.54) (end 88.6 84.44) (width 0.5) (layer "B.Cu") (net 2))
 (segment (start 98.76 121.348478) (end 112.5 135.088478) (width 0.5) (layer "B.Cu") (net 2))
 (segment (start 88.6 110.9) (end 88.735 110.765) (width 0.5) (layer "B.Cu") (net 2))
 (segment (start 120.5 136.25) (end 123 138.75) (width 0.5) (layer "B.Cu") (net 2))
 (segment (start 105.23 125.98) (end 118 138.75) (width 0.5) (layer "B.Cu") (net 6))
 (segment (start 91.5 91.7) (end 105.23 105.43) (width 0.5) (layer "B.Cu") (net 6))
 (segment (start 105.23 105.43) (end 105.23 125.98) (width 0.5) (layer "B.Cu") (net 6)))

